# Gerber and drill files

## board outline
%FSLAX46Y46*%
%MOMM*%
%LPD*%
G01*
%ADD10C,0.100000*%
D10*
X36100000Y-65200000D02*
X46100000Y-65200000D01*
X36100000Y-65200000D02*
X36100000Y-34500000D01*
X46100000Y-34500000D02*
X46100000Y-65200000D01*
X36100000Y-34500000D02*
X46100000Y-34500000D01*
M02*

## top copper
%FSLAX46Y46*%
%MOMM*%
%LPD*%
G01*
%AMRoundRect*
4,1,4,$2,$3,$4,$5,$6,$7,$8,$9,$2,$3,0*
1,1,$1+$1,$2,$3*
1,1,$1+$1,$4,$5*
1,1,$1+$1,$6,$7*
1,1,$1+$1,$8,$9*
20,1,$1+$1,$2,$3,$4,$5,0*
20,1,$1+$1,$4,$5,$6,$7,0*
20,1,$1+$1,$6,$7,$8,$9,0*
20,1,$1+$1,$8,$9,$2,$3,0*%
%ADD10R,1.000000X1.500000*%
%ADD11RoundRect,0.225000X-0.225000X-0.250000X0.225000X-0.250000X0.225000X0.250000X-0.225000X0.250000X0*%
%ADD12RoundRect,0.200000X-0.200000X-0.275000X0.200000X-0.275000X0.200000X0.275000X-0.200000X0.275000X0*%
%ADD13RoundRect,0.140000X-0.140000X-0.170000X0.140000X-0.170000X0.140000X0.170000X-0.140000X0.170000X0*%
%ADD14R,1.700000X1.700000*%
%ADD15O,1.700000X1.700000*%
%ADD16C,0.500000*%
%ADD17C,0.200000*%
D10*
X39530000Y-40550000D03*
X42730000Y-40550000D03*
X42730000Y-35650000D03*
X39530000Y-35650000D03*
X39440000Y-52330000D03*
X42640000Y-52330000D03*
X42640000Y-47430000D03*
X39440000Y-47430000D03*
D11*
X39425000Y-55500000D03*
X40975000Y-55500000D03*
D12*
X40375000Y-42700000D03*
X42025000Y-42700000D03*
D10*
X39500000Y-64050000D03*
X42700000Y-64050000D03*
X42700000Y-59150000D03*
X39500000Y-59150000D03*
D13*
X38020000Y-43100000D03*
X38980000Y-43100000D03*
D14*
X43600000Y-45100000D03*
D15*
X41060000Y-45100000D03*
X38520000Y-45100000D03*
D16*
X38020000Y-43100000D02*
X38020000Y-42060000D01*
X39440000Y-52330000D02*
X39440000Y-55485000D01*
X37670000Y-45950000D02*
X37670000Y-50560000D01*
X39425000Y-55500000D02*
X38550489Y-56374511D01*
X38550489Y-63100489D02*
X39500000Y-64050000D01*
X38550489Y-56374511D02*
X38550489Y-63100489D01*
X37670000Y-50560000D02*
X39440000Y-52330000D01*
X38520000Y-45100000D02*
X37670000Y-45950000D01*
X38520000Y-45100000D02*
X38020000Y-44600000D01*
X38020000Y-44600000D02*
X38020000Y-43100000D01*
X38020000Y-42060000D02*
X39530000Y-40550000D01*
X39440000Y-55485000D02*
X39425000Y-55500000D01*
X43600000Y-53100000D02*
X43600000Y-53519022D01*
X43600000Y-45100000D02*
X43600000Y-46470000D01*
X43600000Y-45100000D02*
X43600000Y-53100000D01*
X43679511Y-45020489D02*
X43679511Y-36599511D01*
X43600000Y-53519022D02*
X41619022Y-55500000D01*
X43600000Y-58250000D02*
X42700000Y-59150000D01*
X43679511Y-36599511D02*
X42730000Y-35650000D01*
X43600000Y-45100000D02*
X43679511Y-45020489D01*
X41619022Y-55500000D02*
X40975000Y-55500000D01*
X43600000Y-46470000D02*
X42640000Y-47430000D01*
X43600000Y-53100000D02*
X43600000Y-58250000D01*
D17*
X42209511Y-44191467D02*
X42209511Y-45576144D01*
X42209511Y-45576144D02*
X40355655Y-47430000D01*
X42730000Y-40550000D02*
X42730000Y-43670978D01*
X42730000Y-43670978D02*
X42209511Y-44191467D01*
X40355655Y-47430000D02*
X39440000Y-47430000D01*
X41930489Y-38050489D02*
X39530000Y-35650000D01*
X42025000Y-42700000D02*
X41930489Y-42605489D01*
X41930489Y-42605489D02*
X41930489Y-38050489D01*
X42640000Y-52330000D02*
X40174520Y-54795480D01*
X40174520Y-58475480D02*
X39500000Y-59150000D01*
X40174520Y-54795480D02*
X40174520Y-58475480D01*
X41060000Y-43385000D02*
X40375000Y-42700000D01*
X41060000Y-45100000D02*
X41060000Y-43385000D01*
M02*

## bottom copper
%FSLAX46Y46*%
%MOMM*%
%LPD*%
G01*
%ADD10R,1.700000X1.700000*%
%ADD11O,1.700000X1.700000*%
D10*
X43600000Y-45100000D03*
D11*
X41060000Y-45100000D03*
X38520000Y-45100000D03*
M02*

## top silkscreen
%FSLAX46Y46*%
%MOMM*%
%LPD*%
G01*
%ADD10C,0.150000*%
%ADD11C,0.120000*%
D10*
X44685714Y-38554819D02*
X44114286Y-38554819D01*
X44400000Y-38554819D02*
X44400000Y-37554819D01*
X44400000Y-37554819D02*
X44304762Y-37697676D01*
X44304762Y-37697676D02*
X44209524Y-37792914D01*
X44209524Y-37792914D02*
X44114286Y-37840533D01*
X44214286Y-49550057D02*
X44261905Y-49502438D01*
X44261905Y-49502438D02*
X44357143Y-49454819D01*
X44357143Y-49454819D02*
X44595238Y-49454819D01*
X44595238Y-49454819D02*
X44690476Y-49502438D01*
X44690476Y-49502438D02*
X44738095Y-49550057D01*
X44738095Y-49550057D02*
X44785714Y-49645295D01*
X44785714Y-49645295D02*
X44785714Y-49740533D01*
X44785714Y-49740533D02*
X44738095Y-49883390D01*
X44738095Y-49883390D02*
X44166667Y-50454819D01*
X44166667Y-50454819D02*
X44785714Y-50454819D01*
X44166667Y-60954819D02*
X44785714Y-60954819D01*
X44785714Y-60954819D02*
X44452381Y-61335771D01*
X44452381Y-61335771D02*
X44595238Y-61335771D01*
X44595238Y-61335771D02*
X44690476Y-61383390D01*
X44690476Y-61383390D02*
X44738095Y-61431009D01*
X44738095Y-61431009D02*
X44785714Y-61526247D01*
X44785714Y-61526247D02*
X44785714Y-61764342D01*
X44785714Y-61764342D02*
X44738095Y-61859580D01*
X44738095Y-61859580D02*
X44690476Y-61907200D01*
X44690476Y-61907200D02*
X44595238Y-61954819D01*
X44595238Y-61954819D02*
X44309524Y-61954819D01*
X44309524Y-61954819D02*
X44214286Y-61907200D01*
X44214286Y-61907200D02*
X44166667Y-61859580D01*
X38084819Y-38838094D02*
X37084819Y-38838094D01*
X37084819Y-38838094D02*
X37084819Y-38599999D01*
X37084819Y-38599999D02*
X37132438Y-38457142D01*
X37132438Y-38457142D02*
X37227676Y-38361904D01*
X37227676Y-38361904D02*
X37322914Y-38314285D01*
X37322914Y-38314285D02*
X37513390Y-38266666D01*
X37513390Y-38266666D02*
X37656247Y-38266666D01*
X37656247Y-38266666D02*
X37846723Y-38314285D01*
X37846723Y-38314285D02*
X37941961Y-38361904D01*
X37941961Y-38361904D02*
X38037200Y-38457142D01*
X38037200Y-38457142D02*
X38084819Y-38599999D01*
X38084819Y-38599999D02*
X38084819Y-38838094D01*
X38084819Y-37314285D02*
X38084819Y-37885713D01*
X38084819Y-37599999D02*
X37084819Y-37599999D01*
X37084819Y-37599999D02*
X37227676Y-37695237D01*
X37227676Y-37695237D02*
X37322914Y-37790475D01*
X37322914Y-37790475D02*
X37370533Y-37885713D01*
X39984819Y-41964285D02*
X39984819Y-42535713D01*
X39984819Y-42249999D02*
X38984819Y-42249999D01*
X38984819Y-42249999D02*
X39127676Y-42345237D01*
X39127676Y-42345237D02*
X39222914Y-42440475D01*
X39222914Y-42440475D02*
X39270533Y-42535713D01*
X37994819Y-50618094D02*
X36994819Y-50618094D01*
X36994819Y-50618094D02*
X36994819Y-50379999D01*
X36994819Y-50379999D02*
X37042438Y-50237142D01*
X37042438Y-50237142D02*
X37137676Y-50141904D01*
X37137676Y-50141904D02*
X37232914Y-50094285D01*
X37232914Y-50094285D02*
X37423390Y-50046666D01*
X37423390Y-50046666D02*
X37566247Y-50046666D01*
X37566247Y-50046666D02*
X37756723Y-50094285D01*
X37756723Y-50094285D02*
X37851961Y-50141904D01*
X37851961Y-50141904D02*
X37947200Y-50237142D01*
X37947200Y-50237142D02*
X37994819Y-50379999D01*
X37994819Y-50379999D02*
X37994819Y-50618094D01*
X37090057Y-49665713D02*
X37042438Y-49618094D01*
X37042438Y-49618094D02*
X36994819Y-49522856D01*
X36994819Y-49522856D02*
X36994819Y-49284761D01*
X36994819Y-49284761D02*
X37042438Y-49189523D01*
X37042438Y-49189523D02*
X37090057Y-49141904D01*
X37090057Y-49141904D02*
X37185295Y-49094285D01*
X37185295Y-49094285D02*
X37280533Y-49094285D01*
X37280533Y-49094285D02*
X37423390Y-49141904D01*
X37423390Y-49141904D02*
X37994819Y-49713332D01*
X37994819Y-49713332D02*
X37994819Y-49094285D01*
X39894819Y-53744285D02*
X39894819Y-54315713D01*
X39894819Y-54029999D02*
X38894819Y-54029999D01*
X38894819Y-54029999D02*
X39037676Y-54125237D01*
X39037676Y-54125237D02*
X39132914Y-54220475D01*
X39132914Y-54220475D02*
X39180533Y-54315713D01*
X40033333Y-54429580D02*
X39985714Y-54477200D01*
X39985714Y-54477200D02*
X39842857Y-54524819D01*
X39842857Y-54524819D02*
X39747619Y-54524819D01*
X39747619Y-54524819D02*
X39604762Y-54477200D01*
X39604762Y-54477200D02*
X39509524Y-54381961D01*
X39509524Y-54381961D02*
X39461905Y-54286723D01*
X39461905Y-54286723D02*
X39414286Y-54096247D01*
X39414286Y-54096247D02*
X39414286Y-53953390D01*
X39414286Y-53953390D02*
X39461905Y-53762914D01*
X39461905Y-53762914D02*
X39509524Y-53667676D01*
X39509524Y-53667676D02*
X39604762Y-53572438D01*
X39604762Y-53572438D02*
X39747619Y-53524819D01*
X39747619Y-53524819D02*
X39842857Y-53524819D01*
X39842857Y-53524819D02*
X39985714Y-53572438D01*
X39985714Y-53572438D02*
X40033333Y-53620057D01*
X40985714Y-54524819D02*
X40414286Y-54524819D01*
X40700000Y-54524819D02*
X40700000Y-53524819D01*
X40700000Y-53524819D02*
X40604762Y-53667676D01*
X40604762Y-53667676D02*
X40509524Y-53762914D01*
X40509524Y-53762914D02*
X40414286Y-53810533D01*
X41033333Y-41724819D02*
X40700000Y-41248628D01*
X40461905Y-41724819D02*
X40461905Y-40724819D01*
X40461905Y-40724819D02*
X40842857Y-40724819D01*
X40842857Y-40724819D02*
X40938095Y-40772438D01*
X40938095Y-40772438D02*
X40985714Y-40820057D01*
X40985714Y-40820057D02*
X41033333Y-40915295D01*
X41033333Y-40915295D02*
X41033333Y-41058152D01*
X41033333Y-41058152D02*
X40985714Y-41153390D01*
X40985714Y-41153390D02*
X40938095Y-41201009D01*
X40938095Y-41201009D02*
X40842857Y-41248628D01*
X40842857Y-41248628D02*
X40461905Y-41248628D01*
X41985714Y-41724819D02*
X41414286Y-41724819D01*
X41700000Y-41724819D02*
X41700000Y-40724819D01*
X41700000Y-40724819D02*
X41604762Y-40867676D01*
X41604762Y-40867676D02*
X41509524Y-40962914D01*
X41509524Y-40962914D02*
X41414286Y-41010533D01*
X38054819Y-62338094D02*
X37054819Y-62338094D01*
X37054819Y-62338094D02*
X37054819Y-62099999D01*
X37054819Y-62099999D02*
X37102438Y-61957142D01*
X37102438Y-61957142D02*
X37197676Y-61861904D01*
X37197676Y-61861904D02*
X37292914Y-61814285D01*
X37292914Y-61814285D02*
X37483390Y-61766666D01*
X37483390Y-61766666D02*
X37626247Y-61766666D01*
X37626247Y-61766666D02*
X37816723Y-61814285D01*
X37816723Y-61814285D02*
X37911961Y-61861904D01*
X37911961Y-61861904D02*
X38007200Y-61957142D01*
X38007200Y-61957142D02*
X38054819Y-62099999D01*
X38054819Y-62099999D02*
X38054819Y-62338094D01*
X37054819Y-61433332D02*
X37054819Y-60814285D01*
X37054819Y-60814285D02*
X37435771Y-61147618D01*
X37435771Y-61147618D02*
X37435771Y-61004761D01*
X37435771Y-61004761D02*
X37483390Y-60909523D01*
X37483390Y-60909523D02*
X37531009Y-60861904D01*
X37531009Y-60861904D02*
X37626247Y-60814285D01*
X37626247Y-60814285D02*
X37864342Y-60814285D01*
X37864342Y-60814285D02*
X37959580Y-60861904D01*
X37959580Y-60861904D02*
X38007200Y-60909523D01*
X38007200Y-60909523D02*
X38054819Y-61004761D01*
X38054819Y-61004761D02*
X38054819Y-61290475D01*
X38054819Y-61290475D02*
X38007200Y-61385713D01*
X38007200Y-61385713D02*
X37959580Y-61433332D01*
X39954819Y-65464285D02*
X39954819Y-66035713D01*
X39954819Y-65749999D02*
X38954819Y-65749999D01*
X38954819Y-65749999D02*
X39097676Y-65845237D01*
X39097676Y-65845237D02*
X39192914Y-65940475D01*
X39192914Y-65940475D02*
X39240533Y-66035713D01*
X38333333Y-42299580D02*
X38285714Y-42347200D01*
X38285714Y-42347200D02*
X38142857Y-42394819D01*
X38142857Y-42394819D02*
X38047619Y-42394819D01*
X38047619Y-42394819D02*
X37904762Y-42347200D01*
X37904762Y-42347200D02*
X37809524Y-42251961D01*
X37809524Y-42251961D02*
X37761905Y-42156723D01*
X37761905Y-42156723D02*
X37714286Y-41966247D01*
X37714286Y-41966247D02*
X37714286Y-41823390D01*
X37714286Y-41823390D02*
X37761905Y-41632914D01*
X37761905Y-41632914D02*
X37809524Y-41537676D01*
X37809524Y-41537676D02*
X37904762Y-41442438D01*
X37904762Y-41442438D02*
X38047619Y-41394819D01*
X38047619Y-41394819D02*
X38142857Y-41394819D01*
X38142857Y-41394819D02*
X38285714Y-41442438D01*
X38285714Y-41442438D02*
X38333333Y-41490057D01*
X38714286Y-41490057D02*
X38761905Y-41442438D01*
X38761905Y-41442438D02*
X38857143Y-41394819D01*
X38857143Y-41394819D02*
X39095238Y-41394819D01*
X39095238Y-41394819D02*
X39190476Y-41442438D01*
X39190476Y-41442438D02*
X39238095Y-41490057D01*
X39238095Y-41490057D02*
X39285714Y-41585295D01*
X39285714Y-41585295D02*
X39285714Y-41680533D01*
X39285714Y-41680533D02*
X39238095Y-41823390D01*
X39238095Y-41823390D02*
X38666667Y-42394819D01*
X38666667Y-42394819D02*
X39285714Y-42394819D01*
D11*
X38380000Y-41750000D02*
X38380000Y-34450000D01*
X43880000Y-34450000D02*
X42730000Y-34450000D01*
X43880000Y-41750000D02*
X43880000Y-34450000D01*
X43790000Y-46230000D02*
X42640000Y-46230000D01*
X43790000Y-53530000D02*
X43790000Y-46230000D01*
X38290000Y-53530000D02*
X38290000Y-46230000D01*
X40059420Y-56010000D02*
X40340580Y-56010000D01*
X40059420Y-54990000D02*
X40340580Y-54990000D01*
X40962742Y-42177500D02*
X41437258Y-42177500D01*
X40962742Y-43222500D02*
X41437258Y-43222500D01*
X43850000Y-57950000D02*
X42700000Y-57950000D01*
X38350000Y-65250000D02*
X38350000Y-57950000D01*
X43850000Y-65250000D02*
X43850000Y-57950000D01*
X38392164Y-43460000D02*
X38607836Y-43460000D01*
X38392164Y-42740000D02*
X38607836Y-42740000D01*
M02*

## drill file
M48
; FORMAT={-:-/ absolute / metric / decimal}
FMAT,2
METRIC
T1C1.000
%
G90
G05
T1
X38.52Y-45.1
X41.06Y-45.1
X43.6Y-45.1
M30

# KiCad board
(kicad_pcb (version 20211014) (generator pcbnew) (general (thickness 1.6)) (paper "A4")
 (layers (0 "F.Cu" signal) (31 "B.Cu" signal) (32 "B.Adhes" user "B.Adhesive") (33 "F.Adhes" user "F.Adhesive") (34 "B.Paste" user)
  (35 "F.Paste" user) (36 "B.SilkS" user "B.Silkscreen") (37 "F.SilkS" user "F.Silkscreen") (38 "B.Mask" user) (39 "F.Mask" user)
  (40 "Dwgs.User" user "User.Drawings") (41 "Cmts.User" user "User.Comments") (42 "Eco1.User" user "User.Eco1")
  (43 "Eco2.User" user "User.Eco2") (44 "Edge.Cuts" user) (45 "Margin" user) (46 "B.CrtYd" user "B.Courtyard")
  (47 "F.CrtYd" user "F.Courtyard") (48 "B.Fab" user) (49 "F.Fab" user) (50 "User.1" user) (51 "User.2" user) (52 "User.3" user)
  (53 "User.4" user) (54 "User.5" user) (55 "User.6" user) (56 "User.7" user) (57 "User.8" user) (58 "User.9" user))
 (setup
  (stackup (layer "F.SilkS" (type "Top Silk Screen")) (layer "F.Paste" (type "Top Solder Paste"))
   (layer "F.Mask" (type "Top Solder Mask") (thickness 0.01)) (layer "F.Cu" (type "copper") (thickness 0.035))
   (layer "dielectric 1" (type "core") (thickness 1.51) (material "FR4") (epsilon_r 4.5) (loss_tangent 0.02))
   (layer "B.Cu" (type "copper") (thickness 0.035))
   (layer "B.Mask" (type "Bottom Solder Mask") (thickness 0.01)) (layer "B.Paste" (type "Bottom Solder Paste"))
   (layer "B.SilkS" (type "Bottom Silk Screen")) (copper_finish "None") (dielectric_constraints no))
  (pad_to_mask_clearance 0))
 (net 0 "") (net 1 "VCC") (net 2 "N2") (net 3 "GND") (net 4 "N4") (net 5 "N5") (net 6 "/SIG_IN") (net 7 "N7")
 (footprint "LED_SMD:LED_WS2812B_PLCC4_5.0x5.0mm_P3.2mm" (layer "F.Cu") (at 41.13 38.1 90)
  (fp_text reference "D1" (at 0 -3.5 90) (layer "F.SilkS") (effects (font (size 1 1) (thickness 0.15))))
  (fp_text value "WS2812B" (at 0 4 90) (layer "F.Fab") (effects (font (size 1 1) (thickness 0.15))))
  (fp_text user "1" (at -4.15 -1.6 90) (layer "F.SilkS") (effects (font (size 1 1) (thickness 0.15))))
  (fp_line (start -3.65 -2.75) (end 3.65 -2.75) (layer "F.SilkS") (width 0.12))
  (fp_line (start 3.65 2.75) (end 3.65 1.6) (layer "F.SilkS") (width 0.12))
  (fp_line (start -3.65 2.75) (end 3.65 2.75) (layer "F.SilkS") (width 0.12))
  (pad "1" smd rect (at -2.45 -1.6 90) (size 1.5 1) (layers "F.Cu" "F.Paste" "F.Mask") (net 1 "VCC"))
  (pad "2" smd rect (at -2.45 1.6 90) (size 1.5 1) (layers "F.Cu" "F.Paste" "F.Mask") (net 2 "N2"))
  (pad "3" smd rect (at 2.45 1.6 90) (size 1.5 1) (layers "F.Cu" "F.Paste" "F.Mask") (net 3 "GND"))
  (pad "4" smd rect (at 2.45 -1.6 90) (size 1.5 1) (layers "F.Cu" "F.Paste" "F.Mask") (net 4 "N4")))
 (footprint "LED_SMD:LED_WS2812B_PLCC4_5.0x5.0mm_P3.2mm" (layer "F.Cu") (at 41.04 49.88 90)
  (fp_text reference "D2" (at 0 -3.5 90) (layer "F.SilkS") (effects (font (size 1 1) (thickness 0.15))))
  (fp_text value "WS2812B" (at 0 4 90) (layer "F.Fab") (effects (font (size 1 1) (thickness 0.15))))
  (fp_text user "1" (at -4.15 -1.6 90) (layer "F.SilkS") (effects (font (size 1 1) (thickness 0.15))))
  (fp_line (start 3.65 2.75) (end 3.65 1.6) (layer "F.SilkS") (width 0.12))
  (fp_line (start -3.65 2.75) (end 3.65 2.75) (layer "F.SilkS") (width 0.12))
  (fp_line (start -3.65 -2.75) (end 3.65 -2.75) (layer "F.SilkS") (width 0.12))
  (pad "1" smd rect (at -2.45 -1.6 90) (size 1.5 1) (layers "F.Cu" "F.Paste" "F.Mask") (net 1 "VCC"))
  (pad "2" smd rect (at -2.45 1.6 90) (size 1.5 1) (layers "F.Cu" "F.Paste" "F.Mask") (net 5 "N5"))
  (pad "3" smd rect (at 2.45 1.6 90) (size 1.5 1) (layers "F.Cu" "F.Paste" "F.Mask") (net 3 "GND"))
  (pad "4" smd rect (at 2.45 -1.6 90) (size 1.5 1) (layers "F.Cu" "F.Paste" "F.Mask") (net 2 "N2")))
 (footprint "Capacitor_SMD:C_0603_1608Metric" (layer "F.Cu") (at 40.2 55.5)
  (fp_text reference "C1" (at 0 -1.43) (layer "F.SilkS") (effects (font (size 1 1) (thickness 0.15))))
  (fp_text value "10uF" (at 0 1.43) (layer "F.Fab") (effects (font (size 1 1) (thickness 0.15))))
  (fp_line (start -0.14058 0.51) (end 0.14058 0.51) (layer "F.SilkS") (width 0.12))
  (fp_line (start -0.14058 -0.51) (end 0.14058 -0.51) (layer "F.SilkS") (width 0.12))
  (pad "1" smd roundrect (at -0.775 0) (size 0.9 0.95) (layers "F.Cu" "F.Paste" "F.Mask") (roundrect_rratio 0.25) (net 1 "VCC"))
  (pad "2" smd roundrect (at 0.775 0) (size 0.9 0.95) (layers "F.Cu" "F.Paste" "F.Mask") (roundrect_rratio 0.25) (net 3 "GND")))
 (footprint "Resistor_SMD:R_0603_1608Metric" (layer "F.Cu") (at 41.2 42.7)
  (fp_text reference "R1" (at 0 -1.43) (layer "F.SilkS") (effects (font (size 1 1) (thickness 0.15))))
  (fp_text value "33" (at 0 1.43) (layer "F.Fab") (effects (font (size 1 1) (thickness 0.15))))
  (fp_line (start -0.237258 -0.5225) (end 0.237258 -0.5225) (layer "F.SilkS") (width 0.12))
  (fp_line (start -0.237258 0.5225) (end 0.237258 0.5225) (layer "F.SilkS") (width 0.12))
  (pad "1" smd roundrect (at -0.825 0) (size 0.8 0.95) (layers "F.Cu" "F.Paste" "F.Mask") (roundrect_rratio 0.25) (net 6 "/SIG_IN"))
  (pad "2" smd roundrect (at 0.825 0) (size 0.8 0.95) (layers "F.Cu" "F.Paste" "F.Mask") (roundrect_rratio 0.25) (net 4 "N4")))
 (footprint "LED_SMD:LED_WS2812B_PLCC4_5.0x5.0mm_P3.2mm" (layer "F.Cu") (at 41.1 61.6 90)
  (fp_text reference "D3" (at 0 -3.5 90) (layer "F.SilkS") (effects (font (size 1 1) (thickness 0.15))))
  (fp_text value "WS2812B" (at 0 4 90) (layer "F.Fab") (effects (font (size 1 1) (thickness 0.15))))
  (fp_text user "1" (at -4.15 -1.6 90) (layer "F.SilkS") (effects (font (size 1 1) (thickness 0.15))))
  (fp_line (start 3.65 2.75) (end 3.65 1.6) (layer "F.SilkS") (width 0.12))
  (fp_line (start -3.65 -2.75) (end 3.65 -2.75) (layer "F.SilkS") (width 0.12))
  (fp_line (start -3.65 2.75) (end 3.65 2.75) (layer "F.SilkS") (width 0.12))
  (pad "1" smd rect (at -2.45 -1.6 90) (size 1.5 1) (layers "F.Cu" "F.Paste" "F.Mask") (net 1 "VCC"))
  (pad "2" smd rect (at -2.45 1.6 90) (size 1.5 1) (layers "F.Cu" "F.Paste" "F.Mask") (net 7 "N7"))
  (pad "3" smd rect (at 2.45 1.6 90) (size 1.5 1) (layers "F.Cu" "F.Paste" "F.Mask") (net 3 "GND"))
  (pad "4" smd rect (at 2.45 -1.6 90) (size 1.5 1) (layers "F.Cu" "F.Paste" "F.Mask") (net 5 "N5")))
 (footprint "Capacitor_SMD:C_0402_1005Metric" (layer "F.Cu") (at 38.5 43.1)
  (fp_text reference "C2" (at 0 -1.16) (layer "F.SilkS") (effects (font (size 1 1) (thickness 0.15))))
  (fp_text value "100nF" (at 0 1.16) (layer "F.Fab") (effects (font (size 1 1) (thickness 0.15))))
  (fp_line (start -0.107836 0.36) (end 0.107836 0.36) (layer "F.SilkS") (width 0.12))
  (fp_line (start -0.107836 -0.36) (end 0.107836 -0.36) (layer "F.SilkS") (width 0.12))
  (pad "1" smd roundrect (at -0.48 0) (size 0.56 0.62) (layers "F.Cu" "F.Paste" "F.Mask") (roundrect_rratio 0.25) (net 1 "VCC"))
  (pad "2" smd roundrect (at 0.48 0) (size 0.56 0.62) (layers "F.Cu" "F.Paste" "F.Mask") (roundrect_rratio 0.25) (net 3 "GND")))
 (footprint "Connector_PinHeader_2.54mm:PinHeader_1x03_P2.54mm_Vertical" (layer "B.Cu") (at 43.6 45.1 90)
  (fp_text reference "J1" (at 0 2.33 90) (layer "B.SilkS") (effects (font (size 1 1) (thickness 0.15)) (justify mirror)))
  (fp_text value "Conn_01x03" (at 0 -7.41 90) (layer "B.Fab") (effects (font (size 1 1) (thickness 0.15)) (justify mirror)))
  (pad "1" thru_hole rect (at 0 0 90) (size 1.7 1.7) (drill 1) (layers *.Cu *.Mask) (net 3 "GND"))
  (pad "2" thru_hole oval (at 0 -2.54 90) (size 1.7 1.7) (drill 1) (layers *.Cu *.Mask) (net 6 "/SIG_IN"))
  (pad "3" thru_hole oval (at 0 -5.08 90) (size 1.7 1.7) (drill 1) (layers *.Cu *.Mask) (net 1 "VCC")))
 (gr_line (start 36.1 65.2) (end 46.1 65.2) (layer "Edge.Cuts") (width 0.1))
 (gr_line (start 36.1 65.2) (end 36.1 34.5) (layer "Edge.Cuts") (width 0.1))
 (gr_line (start 46.1 34.5) (end 46.1 65.2) (layer "Edge.Cuts") (width 0.1))
 (gr_line (start 36.1 34.5) (end 46.1 34.5) (layer "Edge.Cuts") (width 0.1))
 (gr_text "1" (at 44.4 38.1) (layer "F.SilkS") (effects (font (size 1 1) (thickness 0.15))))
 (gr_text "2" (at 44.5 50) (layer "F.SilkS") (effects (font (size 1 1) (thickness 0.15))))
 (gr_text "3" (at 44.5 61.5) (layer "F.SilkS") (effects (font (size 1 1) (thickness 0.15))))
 (segment (start 38.02 43.1) (end 38.02 42.06) (width 0.5) (layer "F.Cu") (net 1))
 (segment (start 39.44 52.33) (end 39.44 55.485) (width 0.5) (layer "F.Cu") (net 1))
 (segment (start 37.67 45.95) (end 37.67 50.56) (width 0.5) (layer "F.Cu") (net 1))
 (segment (start 39.425 55.5) (end 38.550489 56.374511) (width 0.5) (layer "F.Cu") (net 1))
 (segment (start 38.550489 63.100489) (end 39.5 64.05) (width 0.5) (layer "F.Cu") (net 1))
 (segment (start 38.550489 56.374511) (end 38.550489 63.100489) (width 0.5) (layer "F.Cu") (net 1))
 (segment (start 37.67 50.56) (end 39.44 52.33) (width 0.5) (layer "F.Cu") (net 1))
 (segment (start 38.52 45.1) (end 37.67 45.95) (width 0.5) (layer "F.Cu") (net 1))
 (segment (start 38.52 45.1) (end 38.02 44.6) (width 0.5) (layer "F.Cu") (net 1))
 (segment (start 38.02 44.6) (end 38.02 43.1) (width 0.5) (layer "F.Cu") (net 1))
 (segment (start 38.02 42.06) (end 39.53 40.55) (width 0.5) (layer "F.Cu") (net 1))
 (segment (start 39.44 55.485) (end 39.425 55.5) (width 0.5) (layer "F.Cu") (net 1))
 (segment (start 43.6 53.1) (end 43.6 53.519022) (width 0.5) (layer "F.Cu") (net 3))
 (segment (start 43.6 45.1) (end 43.6 46.47) (width 0.5) (layer "F.Cu") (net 3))
 (segment (start 43.6 45.1) (end 43.6 53.1) (width 0.5) (layer "F.Cu") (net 3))
 (segment (start 43.679511 45.020489) (end 43.679511 36.599511) (width 0.5) (layer "F.Cu") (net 3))
 (segment (start 43.6 53.519022) (end 41.619022 55.5) (width 0.5) (layer "F.Cu") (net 3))
 (segment (start 43.6 58.25) (end 42.7 59.15) (width 0.5) (layer "F.Cu") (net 3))
 (segment (start 43.679511 36.599511) (end 42.73 35.65) (width 0.5) (layer "F.Cu") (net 3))
 (segment (start 43.6 45.1) (end 43.679511 45.020489) (width 0.5) (layer "F.Cu") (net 3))
 (segment (start 41.619022 55.5) (end 40.975 55.5) (width 0.5) (layer "F.Cu") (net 3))
 (segment (start 43.6 46.47) (end 42.64 47.43) (width 0.5) (layer "F.Cu") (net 3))
 (segment (start 43.6 53.1) (end 43.6 58.25) (width 0.5) (layer "F.Cu") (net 3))
 (segment (start 42.209511 44.191467) (end 42.209511 45.576144) (width 0.2) (layer "F.Cu") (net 2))
 (segment (start 42.209511 45.576144) (end 40.355655 47.43) (width 0.2) (layer "F.Cu") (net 2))
 (segment (start 42.73 40.55) (end 42.73 43.670978) (width 0.2) (layer "F.Cu") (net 2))
 (segment (start 42.73 43.670978) (end 42.209511 44.191467) (width 0.2) (layer "F.Cu") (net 2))
 (segment (start 40.355655 47.43) (end 39.44 47.43) (width 0.2) (layer "F.Cu") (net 2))
 (segment (start 41.930489 38.050489) (end 39.53 35.65) (width 0.2) (layer "F.Cu") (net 4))
 (segment (start 42.025 42.7) (end 41.930489 42.605489) (width 0.2) (layer "F.Cu") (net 4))
 (segment (start 41.930489 42.605489) (end 41.930489 38.050489) (width 0.2) (layer "F.Cu") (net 4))
 (segment (start 42.64 52.33) (end 40.17452 54.79548) (width 0.2) (layer "F.Cu") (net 5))
 (segment (start 40.17452 58.47548) (end 39.5 59.15) (width 0.2) (layer "F.Cu") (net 5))
 (segment (start 40.17452 54.79548) (end 40.17452 58.47548) (width 0.2) (layer "F.Cu") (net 5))
 (segment (start 41.06 43.385) (end 40.375 42.7) (width 0.2) (layer "F.Cu") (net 6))
 (segment (start 41.06 45.1) (end 41.06 43.385) (width 0.2) (layer "F.Cu") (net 6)))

